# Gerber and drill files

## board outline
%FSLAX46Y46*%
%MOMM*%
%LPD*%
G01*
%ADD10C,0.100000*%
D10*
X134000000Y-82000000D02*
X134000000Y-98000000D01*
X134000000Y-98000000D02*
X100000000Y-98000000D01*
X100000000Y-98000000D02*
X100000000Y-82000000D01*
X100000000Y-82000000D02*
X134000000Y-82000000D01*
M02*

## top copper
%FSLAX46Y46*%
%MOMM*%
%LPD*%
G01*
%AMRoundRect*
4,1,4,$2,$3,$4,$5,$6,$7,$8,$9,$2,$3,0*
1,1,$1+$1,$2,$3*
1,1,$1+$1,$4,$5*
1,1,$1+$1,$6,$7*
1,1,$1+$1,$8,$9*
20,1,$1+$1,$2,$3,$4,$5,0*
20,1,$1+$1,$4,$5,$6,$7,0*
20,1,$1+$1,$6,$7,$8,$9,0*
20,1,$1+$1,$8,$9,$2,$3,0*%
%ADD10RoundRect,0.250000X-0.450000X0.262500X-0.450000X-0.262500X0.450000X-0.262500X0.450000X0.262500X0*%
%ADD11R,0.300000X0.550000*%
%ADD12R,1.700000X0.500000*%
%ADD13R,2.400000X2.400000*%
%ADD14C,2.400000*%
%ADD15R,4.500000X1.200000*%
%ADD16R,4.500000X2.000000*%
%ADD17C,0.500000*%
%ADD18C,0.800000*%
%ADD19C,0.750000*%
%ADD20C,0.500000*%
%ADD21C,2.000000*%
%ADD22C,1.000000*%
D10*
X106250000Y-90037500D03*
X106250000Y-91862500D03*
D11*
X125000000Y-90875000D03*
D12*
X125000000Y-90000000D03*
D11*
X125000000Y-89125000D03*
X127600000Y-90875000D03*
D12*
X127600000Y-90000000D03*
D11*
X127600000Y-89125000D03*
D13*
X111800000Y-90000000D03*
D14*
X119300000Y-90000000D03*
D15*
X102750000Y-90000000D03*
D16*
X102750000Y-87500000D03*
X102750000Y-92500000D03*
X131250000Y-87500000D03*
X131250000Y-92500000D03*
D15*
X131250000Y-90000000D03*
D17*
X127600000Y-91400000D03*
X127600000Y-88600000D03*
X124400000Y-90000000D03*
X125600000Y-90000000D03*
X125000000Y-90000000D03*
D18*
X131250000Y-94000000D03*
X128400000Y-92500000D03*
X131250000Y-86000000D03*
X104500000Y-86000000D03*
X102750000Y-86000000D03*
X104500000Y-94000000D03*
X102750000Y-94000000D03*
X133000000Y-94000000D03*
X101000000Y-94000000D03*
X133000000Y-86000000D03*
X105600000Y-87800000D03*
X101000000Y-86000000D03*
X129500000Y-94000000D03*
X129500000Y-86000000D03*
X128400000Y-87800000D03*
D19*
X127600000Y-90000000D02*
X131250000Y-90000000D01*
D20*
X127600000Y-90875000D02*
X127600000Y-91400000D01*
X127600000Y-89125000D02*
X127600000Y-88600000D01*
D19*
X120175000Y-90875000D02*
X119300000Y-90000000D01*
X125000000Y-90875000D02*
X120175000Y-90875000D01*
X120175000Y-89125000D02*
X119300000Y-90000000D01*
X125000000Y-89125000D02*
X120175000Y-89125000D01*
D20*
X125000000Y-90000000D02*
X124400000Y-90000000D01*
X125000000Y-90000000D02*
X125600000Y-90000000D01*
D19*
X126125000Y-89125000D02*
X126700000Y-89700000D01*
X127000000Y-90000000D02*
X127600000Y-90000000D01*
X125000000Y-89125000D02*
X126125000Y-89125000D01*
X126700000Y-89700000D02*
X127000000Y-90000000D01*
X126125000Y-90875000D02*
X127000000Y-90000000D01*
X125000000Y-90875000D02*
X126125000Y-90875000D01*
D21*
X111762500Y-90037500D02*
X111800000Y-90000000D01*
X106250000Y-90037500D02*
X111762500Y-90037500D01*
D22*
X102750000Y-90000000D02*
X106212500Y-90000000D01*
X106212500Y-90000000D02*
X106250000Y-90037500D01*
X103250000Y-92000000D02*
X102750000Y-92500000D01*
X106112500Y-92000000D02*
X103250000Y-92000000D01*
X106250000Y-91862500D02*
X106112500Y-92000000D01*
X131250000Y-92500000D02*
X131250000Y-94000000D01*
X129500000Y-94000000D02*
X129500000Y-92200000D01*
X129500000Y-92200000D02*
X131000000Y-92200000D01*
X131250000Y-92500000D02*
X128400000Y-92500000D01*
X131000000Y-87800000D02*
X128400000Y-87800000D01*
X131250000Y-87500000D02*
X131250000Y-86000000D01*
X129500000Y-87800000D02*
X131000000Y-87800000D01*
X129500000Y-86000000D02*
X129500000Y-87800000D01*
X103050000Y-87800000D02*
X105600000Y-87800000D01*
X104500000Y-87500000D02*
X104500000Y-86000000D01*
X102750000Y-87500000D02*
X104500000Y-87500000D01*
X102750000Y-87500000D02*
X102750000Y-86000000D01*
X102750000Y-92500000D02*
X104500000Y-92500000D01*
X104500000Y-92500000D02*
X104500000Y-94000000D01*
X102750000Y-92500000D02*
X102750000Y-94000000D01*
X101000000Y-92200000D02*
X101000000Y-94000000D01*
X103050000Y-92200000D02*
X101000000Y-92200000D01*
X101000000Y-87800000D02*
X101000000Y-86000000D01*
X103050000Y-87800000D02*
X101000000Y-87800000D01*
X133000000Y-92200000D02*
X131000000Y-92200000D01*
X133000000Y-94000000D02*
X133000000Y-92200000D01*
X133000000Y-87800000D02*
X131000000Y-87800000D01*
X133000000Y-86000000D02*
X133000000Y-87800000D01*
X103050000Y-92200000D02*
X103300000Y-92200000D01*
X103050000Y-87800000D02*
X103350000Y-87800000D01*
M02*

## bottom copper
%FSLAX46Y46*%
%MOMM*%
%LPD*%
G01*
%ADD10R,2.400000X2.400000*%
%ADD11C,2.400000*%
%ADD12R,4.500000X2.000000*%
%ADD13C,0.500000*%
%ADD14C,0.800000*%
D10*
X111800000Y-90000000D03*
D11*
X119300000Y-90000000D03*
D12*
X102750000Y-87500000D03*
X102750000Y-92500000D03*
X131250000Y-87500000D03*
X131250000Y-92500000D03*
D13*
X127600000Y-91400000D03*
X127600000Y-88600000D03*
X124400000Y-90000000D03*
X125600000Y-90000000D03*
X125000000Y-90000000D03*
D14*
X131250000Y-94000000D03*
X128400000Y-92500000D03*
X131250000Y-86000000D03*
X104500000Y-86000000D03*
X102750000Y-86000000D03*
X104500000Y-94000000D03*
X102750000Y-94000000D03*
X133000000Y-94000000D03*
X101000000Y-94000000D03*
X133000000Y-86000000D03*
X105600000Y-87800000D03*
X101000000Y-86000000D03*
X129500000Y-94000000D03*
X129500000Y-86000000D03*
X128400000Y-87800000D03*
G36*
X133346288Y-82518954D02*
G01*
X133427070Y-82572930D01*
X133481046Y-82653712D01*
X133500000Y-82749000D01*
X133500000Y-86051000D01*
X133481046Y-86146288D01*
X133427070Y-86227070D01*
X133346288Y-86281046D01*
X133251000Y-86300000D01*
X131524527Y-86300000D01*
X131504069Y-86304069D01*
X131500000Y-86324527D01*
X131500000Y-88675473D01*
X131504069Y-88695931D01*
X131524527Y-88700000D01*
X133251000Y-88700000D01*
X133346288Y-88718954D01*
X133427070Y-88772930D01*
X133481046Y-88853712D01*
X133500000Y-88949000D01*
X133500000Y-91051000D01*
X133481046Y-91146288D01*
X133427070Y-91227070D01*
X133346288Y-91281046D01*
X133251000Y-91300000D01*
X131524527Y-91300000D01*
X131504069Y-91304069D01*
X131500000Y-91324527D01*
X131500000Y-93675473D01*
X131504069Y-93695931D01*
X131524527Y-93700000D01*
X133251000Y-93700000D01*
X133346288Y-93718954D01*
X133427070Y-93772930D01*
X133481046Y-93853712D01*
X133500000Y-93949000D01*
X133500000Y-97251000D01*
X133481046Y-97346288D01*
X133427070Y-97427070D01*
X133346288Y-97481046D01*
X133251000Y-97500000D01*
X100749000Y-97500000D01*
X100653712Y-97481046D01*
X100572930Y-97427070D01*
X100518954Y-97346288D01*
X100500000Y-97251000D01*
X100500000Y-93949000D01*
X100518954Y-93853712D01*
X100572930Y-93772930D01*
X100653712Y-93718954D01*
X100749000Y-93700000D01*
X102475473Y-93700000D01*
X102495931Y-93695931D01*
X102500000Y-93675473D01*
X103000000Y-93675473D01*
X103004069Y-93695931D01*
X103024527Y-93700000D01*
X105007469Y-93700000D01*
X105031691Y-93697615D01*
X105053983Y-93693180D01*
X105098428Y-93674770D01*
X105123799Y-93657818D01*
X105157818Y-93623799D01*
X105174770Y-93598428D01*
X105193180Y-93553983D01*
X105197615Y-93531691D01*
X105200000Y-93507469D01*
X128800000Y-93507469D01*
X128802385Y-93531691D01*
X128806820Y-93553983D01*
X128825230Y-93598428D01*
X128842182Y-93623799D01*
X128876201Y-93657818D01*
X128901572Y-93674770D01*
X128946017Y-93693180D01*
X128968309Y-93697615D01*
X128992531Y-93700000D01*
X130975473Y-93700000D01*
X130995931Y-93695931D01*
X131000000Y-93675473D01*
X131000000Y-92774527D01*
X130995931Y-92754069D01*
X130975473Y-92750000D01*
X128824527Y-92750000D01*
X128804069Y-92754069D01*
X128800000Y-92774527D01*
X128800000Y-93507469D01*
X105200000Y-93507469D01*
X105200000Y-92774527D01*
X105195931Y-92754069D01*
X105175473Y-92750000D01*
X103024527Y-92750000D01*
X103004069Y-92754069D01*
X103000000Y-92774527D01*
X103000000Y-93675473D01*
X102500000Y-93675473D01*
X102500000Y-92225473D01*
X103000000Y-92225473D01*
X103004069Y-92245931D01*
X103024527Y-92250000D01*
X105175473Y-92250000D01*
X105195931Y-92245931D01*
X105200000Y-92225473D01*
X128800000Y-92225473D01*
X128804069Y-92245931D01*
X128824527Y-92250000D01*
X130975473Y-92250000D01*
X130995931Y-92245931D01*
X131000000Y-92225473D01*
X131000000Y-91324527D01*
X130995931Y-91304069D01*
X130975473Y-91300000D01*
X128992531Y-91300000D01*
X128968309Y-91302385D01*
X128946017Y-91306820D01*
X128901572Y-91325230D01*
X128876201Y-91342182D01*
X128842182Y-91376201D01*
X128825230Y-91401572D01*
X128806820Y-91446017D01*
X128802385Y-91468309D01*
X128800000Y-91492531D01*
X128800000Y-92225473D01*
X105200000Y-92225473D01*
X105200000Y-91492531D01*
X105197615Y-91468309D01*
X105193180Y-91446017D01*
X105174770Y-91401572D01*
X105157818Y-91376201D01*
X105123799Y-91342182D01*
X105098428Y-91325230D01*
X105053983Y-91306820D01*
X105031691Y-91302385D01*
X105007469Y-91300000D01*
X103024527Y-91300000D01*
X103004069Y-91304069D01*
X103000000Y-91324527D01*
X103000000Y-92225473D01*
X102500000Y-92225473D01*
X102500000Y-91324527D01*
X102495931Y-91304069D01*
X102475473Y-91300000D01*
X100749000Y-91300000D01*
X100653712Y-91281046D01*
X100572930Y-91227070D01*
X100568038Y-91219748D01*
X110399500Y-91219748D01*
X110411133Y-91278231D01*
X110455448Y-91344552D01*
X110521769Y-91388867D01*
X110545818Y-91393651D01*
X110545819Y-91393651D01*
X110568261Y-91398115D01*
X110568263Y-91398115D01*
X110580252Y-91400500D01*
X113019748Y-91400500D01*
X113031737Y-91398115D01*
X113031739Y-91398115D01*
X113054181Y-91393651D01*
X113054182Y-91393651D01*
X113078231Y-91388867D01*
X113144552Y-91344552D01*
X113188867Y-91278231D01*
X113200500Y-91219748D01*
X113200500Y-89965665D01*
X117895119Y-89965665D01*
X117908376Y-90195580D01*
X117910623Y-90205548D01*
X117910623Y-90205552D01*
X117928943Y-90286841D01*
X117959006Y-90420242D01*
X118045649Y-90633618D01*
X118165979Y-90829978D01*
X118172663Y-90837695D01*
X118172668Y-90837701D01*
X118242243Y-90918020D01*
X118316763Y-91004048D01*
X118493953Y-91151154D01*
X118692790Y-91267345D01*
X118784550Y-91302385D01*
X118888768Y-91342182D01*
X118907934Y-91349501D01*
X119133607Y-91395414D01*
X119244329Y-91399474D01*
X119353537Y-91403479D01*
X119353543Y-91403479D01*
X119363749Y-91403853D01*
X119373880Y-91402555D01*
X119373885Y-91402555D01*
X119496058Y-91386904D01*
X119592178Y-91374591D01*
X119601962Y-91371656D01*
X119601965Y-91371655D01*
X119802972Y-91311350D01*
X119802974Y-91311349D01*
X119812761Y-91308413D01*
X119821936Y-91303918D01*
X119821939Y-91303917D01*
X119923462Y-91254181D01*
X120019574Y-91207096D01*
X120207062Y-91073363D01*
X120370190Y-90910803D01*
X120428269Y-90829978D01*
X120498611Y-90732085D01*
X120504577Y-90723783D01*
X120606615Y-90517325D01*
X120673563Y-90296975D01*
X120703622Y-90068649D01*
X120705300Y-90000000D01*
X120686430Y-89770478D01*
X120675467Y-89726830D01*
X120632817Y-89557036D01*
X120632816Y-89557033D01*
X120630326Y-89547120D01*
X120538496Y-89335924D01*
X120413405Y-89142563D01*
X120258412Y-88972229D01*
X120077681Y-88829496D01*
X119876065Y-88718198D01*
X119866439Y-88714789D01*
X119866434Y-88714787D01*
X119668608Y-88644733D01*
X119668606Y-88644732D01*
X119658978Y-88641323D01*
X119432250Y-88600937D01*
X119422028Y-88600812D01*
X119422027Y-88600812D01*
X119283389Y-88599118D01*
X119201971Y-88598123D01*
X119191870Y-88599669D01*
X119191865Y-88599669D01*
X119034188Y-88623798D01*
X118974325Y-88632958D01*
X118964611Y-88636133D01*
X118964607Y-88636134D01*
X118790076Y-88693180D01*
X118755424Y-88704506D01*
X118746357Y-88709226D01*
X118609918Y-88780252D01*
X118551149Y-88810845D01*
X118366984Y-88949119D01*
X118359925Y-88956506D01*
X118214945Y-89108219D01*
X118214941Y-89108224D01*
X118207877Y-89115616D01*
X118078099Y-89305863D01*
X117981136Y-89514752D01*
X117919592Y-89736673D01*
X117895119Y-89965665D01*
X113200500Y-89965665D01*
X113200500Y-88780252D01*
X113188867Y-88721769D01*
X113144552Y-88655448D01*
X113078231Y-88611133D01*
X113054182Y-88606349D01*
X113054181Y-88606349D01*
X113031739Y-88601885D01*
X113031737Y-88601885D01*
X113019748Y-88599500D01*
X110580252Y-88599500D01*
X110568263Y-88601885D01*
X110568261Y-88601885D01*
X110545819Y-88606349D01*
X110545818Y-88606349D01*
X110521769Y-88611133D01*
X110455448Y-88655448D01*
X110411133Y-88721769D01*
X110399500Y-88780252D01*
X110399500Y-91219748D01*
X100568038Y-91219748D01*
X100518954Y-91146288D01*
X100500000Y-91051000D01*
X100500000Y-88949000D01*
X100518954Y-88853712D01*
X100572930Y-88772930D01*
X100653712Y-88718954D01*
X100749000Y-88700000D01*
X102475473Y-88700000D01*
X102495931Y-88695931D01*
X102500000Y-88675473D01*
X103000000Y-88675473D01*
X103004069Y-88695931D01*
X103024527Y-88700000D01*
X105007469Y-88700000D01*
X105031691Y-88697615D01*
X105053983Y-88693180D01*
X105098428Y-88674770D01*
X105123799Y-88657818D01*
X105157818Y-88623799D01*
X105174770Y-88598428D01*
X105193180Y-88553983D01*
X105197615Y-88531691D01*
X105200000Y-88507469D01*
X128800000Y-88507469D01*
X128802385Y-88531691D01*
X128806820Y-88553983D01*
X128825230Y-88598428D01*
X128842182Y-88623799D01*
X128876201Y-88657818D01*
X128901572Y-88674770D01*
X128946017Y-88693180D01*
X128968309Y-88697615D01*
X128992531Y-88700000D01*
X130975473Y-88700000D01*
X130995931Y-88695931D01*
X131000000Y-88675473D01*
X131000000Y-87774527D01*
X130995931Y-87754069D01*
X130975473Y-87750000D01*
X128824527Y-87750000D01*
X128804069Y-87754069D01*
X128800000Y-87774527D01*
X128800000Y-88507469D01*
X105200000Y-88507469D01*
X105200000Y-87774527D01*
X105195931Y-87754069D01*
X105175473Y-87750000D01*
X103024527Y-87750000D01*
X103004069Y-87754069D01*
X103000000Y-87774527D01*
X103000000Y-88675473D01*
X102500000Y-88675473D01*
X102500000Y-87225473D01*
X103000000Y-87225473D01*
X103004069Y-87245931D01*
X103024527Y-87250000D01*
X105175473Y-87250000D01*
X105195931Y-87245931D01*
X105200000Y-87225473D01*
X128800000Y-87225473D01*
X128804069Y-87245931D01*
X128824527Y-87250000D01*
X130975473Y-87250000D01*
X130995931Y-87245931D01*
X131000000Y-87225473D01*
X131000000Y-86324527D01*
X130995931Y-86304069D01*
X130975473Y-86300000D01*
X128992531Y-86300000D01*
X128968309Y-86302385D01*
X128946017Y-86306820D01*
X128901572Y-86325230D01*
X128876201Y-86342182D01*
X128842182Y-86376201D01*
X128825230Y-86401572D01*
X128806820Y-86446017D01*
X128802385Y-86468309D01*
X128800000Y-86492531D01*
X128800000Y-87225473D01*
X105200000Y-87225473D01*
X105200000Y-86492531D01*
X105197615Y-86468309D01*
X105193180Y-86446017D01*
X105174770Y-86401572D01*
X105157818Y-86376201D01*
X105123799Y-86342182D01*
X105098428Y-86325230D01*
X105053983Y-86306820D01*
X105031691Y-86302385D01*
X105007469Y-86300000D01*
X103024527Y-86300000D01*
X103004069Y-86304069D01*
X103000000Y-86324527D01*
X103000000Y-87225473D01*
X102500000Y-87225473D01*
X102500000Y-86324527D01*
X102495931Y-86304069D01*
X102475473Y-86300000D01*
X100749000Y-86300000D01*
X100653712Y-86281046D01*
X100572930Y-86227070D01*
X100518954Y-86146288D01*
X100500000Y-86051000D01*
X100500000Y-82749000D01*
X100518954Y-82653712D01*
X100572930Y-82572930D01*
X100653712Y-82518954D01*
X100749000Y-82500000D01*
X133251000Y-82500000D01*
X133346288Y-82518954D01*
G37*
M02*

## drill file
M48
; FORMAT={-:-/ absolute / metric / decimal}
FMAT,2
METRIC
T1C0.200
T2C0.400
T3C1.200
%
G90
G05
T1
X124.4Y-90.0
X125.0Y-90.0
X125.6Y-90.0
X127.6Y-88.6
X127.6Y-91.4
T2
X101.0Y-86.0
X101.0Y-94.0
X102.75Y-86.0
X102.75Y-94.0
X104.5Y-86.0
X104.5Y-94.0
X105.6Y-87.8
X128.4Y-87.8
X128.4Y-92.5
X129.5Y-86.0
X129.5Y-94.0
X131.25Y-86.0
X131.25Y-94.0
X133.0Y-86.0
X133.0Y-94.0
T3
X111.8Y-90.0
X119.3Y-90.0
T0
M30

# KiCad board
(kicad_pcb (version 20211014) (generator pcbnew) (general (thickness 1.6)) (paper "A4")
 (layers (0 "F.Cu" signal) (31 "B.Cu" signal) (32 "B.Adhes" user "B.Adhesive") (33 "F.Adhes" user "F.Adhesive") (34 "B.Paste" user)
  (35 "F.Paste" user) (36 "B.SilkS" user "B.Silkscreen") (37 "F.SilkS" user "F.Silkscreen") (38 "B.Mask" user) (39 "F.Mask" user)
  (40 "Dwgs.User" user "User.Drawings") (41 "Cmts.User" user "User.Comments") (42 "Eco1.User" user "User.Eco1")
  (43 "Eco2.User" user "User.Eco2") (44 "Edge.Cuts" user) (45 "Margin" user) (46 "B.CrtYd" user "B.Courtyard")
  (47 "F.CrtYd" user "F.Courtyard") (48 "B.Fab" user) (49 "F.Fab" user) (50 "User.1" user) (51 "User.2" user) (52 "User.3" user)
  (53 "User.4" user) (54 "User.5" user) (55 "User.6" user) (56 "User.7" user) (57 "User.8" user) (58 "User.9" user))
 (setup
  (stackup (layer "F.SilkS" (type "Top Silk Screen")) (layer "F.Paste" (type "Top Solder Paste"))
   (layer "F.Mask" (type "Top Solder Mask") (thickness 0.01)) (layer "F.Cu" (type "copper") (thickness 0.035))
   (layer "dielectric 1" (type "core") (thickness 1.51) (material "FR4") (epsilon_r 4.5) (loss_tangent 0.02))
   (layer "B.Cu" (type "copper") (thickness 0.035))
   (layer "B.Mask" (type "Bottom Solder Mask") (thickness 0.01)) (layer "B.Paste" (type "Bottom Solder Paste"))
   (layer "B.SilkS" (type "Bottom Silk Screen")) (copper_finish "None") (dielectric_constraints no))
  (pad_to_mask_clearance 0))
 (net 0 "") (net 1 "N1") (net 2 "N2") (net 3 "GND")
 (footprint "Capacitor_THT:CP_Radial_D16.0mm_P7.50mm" (layer "F.Cu") (at 111.8 90)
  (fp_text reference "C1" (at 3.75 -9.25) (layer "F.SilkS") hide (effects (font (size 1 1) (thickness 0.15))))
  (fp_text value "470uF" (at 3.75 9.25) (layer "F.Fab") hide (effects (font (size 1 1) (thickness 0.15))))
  (pad "1" thru_hole rect (at 0 0) (size 2.4 2.4) (drill 1.2) (layers *.Cu *.Mask) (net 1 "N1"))
  (pad "2" thru_hole circle (at 7.5 0) (size 2.4 2.4) (drill 1.2) (layers *.Cu *.Mask) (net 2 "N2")))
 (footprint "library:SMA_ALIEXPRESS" (layer "F.Cu") (at 100.5 90 90)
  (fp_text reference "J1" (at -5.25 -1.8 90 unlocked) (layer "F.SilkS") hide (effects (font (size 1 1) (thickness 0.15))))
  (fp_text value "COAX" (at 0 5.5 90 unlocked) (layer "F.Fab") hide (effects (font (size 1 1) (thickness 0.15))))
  (pad "1" smd rect (at 0 2.25 90) (size 1.2 4.5) (layers "F.Cu" "F.Paste" "F.Mask") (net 1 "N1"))
  (pad "2" smd rect (at -2.5 2.25 90) (size 2 4.5) (layers "B.Cu" "F.Paste" "B.Mask") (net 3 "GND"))
  (pad "2" smd rect (at 2.5 2.25 90) (size 2 4.5) (layers "B.Cu" "F.Paste" "B.Mask") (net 3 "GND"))
  (pad "2" smd rect (at 2.5 2.25 90) (size 2 4.5) (layers "F.Cu" "F.Paste" "F.Mask") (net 3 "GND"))
  (pad "2" smd rect (at -2.5 2.25 90) (size 2 4.5) (layers "F.Cu" "F.Paste" "F.Mask") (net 3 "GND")))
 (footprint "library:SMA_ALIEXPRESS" (layer "F.Cu") (at 133.5 90 -90)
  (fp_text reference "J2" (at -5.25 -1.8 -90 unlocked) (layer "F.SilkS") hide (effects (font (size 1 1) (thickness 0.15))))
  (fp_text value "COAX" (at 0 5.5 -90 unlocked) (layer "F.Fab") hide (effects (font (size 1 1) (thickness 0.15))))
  (pad "1" smd rect (at 0 2.25 270) (size 1.2 4.5) (layers "F.Cu" "F.Paste" "F.Mask") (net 2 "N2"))
  (pad "2" smd rect (at -2.5 2.25 270) (size 2 4.5) (layers "B.Cu" "F.Paste" "B.Mask") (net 3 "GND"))
  (pad "2" smd rect (at -2.5 2.25 270) (size 2 4.5) (layers "F.Cu" "F.Paste" "F.Mask") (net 3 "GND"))
  (pad "2" smd rect (at 2.5 2.25 270) (size 2 4.5) (layers "F.Cu" "F.Paste" "F.Mask") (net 3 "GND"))
  (pad "2" smd rect (at 2.5 2.25 270) (size 2 4.5) (layers "B.Cu" "F.Paste" "B.Mask") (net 3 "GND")))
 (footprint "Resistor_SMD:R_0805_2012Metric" (layer "F.Cu") (at 106.25 90.95 -90)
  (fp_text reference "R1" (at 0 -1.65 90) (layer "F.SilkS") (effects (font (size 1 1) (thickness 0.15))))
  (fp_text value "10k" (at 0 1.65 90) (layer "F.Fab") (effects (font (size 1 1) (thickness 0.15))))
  (pad "1" smd roundrect (at -0.9125 0 270) (size 1.025 1.4) (layers "F.Cu" "F.Paste" "F.Mask") (roundrect_rratio 0.243902439) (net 1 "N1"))
  (pad "2" smd roundrect (at 0.9125 0 270) (size 1.025 1.4) (layers "F.Cu" "F.Paste" "F.Mask") (roundrect_rratio 0.243902439) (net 3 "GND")))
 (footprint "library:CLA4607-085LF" (layer "F.Cu") (at 127.6 90 90)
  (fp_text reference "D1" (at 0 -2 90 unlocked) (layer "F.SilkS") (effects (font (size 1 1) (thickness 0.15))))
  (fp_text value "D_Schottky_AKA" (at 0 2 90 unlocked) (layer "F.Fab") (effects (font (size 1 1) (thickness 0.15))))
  (pad "1" smd rect (at -0.875 0 90) (size 0.55 0.3) (layers "F.Cu" "F.Paste" "F.Mask") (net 3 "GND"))
  (pad "2" smd rect (at 0 0 90) (size 0.5 1.7) (layers "F.Cu" "F.Paste" "F.Mask") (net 2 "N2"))
  (pad "3" smd rect (at 0.875 0 90) (size 0.55 0.3) (layers "F.Cu" "F.Paste" "F.Mask") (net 3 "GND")))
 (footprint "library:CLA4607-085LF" (layer "F.Cu") (at 125 90 90)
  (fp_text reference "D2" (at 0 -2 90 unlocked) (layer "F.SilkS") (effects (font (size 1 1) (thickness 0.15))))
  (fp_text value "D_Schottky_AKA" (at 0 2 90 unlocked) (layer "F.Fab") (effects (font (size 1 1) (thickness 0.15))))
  (pad "1" smd rect (at -0.875 0 90) (size 0.55 0.3) (layers "F.Cu" "F.Paste" "F.Mask") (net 2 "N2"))
  (pad "2" smd rect (at 0 0 90) (size 0.5 1.7) (layers "F.Cu" "F.Paste" "F.Mask") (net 3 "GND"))
  (pad "3" smd rect (at 0.875 0 90) (size 0.55 0.3) (layers "F.Cu" "F.Paste" "F.Mask") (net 2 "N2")))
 (gr_line (start 134 98) (end 100 98) (layer "Edge.Cuts") (width 0.1))
 (gr_line (start 100 98) (end 100 82) (layer "Edge.Cuts") (width 0.1))
 (gr_line (start 100 82) (end 134 82) (layer "Edge.Cuts") (width 0.1))
 (gr_line (start 134 82) (end 134 98) (layer "Edge.Cuts") (width 0.1))
 (segment (start 106.25 90.0375) (end 111.7625 90.0375) (width 2) (layer "F.Cu") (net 1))
 (segment (start 111.7625 90.0375) (end 111.8 90) (width 2) (layer "F.Cu") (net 1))
 (segment (start 102.75 90) (end 106.2125 90) (width 1) (layer "F.Cu") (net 1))
 (segment (start 106.2125 90) (end 106.25 90.0375) (width 1) (layer "F.Cu") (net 1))
 (segment (start 126.125 90.875) (end 127 90) (width 0.75) (layer "F.Cu") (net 2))
 (segment (start 125 89.125) (end 120.175 89.125) (width 0.75) (layer "F.Cu") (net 2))
 (segment (start 120.175 89.125) (end 119.3 90) (width 0.75) (layer "F.Cu") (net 2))
 (segment (start 125 90.875) (end 126.125 90.875) (width 0.75) (layer "F.Cu") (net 2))
 (segment (start 125 90.875) (end 120.175 90.875) (width 0.75) (layer "F.Cu") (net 2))
 (segment (start 120.175 90.875) (end 119.3 90) (width 0.75) (layer "F.Cu") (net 2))
 (segment (start 125 89.125) (end 126.125 89.125) (width 0.75) (layer "F.Cu") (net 2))
 (segment (start 126.7 89.7) (end 127 90) (width 0.75) (layer "F.Cu") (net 2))
 (segment (start 127.6 90) (end 131.25 90) (width 0.75) (layer "F.Cu") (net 2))
 (segment (start 127 90) (end 127.6 90) (width 0.75) (layer "F.Cu") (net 2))
 (segment (start 126.125 89.125) (end 126.7 89.7) (width 0.75) (layer "F.Cu") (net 2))
 (segment (start 129.5 86) (end 129.5 87.8) (width 1) (layer "F.Cu") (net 3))
 (segment (start 101 87.8) (end 101 86) (width 1) (layer "F.Cu") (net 3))
 (segment (start 133 86) (end 133 87.8) (width 1) (layer "F.Cu") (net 3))
 (segment (start 102.75 87.5) (end 102.75 86) (width 1) (layer "F.Cu") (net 3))
 (segment (start 104.5 87.5) (end 104.5 86) (width 1) (layer "F.Cu") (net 3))
 (segment (start 106.25 91.8625) (end 106.1125 92) (width 1) (layer "F.Cu") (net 3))
 (segment (start 103.25 92) (end 102.75 92.5) (width 1) (layer "F.Cu") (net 3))
 (segment (start 101 92.2) (end 101 94) (width 1) (layer "F.Cu") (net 3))
 (segment (start 125 90) (end 124.4 90) (width 0.5) (layer "F.Cu") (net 3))
 (segment (start 102.75 87.5) (end 104.5 87.5) (width 1) (layer "F.Cu") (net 3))
 (segment (start 125 90) (end 125.6 90) (width 0.5) (layer "F.Cu") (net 3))
 (segment (start 104.5 92.5) (end 104.5 94) (width 1) (layer "F.Cu") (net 3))
 (segment (start 127.6 90.875) (end 127.6 91.4) (width 0.5) (layer "F.Cu") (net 3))
 (segment (start 103.05 92.2) (end 101 92.2) (width 1) (layer "F.Cu") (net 3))
 (segment (start 129.5 94) (end 129.5 92.2) (width 1) (layer "F.Cu") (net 3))
 (segment (start 102.75 92.5) (end 102.75 94) (width 1) (layer "F.Cu") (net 3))
 (segment (start 103.05 92.2) (end 103.3 92.2) (width 1) (layer "F.Cu") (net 3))
 (segment (start 103.05 87.8) (end 103.35 87.8) (width 1) (layer "F.Cu") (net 3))
 (segment (start 131.25 92.5) (end 128.4 92.5) (width 1) (layer "F.Cu") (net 3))
 (segment (start 103.05 87.8) (end 101 87.8) (width 1) (layer "F.Cu") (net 3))
 (segment (start 133 87.8) (end 131 87.8) (width 1) (layer "F.Cu") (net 3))
 (segment (start 127.6 89.125) (end 127.6 88.6) (width 0.5) (layer "F.Cu") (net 3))
 (segment (start 131.25 87.5) (end 131.25 86) (width 1) (layer "F.Cu") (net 3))
 (segment (start 106.1125 92) (end 103.25 92) (width 1) (layer "F.Cu") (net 3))
 (segment (start 129.5 92.2) (end 131 92.2) (width 1) (layer "F.Cu") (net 3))
 (segment (start 103.05 87.8) (end 105.6 87.8) (width 1) (layer "F.Cu") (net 3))
 (segment (start 131 87.8) (end 128.4 87.8) (width 1) (layer "F.Cu") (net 3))
 (segment (start 133 92.2) (end 131 92.2) (width 1) (layer "F.Cu") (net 3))
 (segment (start 129.5 87.8) (end 131 87.8) (width 1) (layer "F.Cu") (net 3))
 (segment (start 133 94) (end 133 92.2) (width 1) (layer "F.Cu") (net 3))
 (segment (start 131.25 92.5) (end 131.25 94) (width 1) (layer "F.Cu") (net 3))
 (segment (start 102.75 92.5) (end 104.5 92.5) (width 1) (layer "F.Cu") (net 3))
 (via (at 104.5 86) (size 0.8) (drill 0.4) (layers "F.Cu" "B.Cu") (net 3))
 (via (at 131.25 86) (size 0.8) (drill 0.4) (layers "F.Cu" "B.Cu") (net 3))
 (via (at 127.6 88.6) (size 0.5) (drill 0.2) (layers "F.Cu" "B.Cu") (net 3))
 (via (at 104.5 94) (size 0.8) (drill 0.4) (layers "F.Cu" "B.Cu") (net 3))
 (via (at 101 94) (size 0.8) (drill 0.4) (layers "F.Cu" "B.Cu") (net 3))
 (via (at 128.4 92.5) (size 0.8) (drill 0.4) (layers "F.Cu" "B.Cu") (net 3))
 (via (at 133 86) (size 0.8) (drill 0.4) (layers "F.Cu" "B.Cu") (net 3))
 (via (at 125.6 90) (size 0.5) (drill 0.2) (layers "F.Cu" "B.Cu") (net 3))
 (via (at 105.6 87.8) (size 0.8) (drill 0.4) (layers "F.Cu" "B.Cu") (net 3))
 (via (at 102.75 94) (size 0.8) (drill 0.4) (layers "F.Cu" "B.Cu") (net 3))
 (via (at 127.6 91.4) (size 0.5) (drill 0.2) (layers "F.Cu" "B.Cu") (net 3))
 (via (at 124.4 90) (size 0.5) (drill 0.2) (layers "F.Cu" "B.Cu") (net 3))
 (via (at 102.75 86) (size 0.8) (drill 0.4) (layers "F.Cu" "B.Cu") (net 3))
 (via (at 101 86) (size 0.8) (drill 0.4) (layers "F.Cu" "B.Cu") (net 3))
 (via (at 129.5 94) (size 0.8) (drill 0.4) (layers "F.Cu" "B.Cu") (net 3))
 (via (at 129.5 86) (size 0.8) (drill 0.4) (layers "F.Cu" "B.Cu") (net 3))
 (via (at 131.25 94) (size 0.8) (drill 0.4) (layers "F.Cu" "B.Cu") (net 3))
 (via (at 133 94) (size 0.8) (drill 0.4) (layers "F.Cu" "B.Cu") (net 3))
 (via (at 125 90) (size 0.5) (drill 0.2) (layers "F.Cu" "B.Cu") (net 3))
 (via (at 128.4 87.8) (size 0.8) (drill 0.4) (layers "F.Cu" "B.Cu") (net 3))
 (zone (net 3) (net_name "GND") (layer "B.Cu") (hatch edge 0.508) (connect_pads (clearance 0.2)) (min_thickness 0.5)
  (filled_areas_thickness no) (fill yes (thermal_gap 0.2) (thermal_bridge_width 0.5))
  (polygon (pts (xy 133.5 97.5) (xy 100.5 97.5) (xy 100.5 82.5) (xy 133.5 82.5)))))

